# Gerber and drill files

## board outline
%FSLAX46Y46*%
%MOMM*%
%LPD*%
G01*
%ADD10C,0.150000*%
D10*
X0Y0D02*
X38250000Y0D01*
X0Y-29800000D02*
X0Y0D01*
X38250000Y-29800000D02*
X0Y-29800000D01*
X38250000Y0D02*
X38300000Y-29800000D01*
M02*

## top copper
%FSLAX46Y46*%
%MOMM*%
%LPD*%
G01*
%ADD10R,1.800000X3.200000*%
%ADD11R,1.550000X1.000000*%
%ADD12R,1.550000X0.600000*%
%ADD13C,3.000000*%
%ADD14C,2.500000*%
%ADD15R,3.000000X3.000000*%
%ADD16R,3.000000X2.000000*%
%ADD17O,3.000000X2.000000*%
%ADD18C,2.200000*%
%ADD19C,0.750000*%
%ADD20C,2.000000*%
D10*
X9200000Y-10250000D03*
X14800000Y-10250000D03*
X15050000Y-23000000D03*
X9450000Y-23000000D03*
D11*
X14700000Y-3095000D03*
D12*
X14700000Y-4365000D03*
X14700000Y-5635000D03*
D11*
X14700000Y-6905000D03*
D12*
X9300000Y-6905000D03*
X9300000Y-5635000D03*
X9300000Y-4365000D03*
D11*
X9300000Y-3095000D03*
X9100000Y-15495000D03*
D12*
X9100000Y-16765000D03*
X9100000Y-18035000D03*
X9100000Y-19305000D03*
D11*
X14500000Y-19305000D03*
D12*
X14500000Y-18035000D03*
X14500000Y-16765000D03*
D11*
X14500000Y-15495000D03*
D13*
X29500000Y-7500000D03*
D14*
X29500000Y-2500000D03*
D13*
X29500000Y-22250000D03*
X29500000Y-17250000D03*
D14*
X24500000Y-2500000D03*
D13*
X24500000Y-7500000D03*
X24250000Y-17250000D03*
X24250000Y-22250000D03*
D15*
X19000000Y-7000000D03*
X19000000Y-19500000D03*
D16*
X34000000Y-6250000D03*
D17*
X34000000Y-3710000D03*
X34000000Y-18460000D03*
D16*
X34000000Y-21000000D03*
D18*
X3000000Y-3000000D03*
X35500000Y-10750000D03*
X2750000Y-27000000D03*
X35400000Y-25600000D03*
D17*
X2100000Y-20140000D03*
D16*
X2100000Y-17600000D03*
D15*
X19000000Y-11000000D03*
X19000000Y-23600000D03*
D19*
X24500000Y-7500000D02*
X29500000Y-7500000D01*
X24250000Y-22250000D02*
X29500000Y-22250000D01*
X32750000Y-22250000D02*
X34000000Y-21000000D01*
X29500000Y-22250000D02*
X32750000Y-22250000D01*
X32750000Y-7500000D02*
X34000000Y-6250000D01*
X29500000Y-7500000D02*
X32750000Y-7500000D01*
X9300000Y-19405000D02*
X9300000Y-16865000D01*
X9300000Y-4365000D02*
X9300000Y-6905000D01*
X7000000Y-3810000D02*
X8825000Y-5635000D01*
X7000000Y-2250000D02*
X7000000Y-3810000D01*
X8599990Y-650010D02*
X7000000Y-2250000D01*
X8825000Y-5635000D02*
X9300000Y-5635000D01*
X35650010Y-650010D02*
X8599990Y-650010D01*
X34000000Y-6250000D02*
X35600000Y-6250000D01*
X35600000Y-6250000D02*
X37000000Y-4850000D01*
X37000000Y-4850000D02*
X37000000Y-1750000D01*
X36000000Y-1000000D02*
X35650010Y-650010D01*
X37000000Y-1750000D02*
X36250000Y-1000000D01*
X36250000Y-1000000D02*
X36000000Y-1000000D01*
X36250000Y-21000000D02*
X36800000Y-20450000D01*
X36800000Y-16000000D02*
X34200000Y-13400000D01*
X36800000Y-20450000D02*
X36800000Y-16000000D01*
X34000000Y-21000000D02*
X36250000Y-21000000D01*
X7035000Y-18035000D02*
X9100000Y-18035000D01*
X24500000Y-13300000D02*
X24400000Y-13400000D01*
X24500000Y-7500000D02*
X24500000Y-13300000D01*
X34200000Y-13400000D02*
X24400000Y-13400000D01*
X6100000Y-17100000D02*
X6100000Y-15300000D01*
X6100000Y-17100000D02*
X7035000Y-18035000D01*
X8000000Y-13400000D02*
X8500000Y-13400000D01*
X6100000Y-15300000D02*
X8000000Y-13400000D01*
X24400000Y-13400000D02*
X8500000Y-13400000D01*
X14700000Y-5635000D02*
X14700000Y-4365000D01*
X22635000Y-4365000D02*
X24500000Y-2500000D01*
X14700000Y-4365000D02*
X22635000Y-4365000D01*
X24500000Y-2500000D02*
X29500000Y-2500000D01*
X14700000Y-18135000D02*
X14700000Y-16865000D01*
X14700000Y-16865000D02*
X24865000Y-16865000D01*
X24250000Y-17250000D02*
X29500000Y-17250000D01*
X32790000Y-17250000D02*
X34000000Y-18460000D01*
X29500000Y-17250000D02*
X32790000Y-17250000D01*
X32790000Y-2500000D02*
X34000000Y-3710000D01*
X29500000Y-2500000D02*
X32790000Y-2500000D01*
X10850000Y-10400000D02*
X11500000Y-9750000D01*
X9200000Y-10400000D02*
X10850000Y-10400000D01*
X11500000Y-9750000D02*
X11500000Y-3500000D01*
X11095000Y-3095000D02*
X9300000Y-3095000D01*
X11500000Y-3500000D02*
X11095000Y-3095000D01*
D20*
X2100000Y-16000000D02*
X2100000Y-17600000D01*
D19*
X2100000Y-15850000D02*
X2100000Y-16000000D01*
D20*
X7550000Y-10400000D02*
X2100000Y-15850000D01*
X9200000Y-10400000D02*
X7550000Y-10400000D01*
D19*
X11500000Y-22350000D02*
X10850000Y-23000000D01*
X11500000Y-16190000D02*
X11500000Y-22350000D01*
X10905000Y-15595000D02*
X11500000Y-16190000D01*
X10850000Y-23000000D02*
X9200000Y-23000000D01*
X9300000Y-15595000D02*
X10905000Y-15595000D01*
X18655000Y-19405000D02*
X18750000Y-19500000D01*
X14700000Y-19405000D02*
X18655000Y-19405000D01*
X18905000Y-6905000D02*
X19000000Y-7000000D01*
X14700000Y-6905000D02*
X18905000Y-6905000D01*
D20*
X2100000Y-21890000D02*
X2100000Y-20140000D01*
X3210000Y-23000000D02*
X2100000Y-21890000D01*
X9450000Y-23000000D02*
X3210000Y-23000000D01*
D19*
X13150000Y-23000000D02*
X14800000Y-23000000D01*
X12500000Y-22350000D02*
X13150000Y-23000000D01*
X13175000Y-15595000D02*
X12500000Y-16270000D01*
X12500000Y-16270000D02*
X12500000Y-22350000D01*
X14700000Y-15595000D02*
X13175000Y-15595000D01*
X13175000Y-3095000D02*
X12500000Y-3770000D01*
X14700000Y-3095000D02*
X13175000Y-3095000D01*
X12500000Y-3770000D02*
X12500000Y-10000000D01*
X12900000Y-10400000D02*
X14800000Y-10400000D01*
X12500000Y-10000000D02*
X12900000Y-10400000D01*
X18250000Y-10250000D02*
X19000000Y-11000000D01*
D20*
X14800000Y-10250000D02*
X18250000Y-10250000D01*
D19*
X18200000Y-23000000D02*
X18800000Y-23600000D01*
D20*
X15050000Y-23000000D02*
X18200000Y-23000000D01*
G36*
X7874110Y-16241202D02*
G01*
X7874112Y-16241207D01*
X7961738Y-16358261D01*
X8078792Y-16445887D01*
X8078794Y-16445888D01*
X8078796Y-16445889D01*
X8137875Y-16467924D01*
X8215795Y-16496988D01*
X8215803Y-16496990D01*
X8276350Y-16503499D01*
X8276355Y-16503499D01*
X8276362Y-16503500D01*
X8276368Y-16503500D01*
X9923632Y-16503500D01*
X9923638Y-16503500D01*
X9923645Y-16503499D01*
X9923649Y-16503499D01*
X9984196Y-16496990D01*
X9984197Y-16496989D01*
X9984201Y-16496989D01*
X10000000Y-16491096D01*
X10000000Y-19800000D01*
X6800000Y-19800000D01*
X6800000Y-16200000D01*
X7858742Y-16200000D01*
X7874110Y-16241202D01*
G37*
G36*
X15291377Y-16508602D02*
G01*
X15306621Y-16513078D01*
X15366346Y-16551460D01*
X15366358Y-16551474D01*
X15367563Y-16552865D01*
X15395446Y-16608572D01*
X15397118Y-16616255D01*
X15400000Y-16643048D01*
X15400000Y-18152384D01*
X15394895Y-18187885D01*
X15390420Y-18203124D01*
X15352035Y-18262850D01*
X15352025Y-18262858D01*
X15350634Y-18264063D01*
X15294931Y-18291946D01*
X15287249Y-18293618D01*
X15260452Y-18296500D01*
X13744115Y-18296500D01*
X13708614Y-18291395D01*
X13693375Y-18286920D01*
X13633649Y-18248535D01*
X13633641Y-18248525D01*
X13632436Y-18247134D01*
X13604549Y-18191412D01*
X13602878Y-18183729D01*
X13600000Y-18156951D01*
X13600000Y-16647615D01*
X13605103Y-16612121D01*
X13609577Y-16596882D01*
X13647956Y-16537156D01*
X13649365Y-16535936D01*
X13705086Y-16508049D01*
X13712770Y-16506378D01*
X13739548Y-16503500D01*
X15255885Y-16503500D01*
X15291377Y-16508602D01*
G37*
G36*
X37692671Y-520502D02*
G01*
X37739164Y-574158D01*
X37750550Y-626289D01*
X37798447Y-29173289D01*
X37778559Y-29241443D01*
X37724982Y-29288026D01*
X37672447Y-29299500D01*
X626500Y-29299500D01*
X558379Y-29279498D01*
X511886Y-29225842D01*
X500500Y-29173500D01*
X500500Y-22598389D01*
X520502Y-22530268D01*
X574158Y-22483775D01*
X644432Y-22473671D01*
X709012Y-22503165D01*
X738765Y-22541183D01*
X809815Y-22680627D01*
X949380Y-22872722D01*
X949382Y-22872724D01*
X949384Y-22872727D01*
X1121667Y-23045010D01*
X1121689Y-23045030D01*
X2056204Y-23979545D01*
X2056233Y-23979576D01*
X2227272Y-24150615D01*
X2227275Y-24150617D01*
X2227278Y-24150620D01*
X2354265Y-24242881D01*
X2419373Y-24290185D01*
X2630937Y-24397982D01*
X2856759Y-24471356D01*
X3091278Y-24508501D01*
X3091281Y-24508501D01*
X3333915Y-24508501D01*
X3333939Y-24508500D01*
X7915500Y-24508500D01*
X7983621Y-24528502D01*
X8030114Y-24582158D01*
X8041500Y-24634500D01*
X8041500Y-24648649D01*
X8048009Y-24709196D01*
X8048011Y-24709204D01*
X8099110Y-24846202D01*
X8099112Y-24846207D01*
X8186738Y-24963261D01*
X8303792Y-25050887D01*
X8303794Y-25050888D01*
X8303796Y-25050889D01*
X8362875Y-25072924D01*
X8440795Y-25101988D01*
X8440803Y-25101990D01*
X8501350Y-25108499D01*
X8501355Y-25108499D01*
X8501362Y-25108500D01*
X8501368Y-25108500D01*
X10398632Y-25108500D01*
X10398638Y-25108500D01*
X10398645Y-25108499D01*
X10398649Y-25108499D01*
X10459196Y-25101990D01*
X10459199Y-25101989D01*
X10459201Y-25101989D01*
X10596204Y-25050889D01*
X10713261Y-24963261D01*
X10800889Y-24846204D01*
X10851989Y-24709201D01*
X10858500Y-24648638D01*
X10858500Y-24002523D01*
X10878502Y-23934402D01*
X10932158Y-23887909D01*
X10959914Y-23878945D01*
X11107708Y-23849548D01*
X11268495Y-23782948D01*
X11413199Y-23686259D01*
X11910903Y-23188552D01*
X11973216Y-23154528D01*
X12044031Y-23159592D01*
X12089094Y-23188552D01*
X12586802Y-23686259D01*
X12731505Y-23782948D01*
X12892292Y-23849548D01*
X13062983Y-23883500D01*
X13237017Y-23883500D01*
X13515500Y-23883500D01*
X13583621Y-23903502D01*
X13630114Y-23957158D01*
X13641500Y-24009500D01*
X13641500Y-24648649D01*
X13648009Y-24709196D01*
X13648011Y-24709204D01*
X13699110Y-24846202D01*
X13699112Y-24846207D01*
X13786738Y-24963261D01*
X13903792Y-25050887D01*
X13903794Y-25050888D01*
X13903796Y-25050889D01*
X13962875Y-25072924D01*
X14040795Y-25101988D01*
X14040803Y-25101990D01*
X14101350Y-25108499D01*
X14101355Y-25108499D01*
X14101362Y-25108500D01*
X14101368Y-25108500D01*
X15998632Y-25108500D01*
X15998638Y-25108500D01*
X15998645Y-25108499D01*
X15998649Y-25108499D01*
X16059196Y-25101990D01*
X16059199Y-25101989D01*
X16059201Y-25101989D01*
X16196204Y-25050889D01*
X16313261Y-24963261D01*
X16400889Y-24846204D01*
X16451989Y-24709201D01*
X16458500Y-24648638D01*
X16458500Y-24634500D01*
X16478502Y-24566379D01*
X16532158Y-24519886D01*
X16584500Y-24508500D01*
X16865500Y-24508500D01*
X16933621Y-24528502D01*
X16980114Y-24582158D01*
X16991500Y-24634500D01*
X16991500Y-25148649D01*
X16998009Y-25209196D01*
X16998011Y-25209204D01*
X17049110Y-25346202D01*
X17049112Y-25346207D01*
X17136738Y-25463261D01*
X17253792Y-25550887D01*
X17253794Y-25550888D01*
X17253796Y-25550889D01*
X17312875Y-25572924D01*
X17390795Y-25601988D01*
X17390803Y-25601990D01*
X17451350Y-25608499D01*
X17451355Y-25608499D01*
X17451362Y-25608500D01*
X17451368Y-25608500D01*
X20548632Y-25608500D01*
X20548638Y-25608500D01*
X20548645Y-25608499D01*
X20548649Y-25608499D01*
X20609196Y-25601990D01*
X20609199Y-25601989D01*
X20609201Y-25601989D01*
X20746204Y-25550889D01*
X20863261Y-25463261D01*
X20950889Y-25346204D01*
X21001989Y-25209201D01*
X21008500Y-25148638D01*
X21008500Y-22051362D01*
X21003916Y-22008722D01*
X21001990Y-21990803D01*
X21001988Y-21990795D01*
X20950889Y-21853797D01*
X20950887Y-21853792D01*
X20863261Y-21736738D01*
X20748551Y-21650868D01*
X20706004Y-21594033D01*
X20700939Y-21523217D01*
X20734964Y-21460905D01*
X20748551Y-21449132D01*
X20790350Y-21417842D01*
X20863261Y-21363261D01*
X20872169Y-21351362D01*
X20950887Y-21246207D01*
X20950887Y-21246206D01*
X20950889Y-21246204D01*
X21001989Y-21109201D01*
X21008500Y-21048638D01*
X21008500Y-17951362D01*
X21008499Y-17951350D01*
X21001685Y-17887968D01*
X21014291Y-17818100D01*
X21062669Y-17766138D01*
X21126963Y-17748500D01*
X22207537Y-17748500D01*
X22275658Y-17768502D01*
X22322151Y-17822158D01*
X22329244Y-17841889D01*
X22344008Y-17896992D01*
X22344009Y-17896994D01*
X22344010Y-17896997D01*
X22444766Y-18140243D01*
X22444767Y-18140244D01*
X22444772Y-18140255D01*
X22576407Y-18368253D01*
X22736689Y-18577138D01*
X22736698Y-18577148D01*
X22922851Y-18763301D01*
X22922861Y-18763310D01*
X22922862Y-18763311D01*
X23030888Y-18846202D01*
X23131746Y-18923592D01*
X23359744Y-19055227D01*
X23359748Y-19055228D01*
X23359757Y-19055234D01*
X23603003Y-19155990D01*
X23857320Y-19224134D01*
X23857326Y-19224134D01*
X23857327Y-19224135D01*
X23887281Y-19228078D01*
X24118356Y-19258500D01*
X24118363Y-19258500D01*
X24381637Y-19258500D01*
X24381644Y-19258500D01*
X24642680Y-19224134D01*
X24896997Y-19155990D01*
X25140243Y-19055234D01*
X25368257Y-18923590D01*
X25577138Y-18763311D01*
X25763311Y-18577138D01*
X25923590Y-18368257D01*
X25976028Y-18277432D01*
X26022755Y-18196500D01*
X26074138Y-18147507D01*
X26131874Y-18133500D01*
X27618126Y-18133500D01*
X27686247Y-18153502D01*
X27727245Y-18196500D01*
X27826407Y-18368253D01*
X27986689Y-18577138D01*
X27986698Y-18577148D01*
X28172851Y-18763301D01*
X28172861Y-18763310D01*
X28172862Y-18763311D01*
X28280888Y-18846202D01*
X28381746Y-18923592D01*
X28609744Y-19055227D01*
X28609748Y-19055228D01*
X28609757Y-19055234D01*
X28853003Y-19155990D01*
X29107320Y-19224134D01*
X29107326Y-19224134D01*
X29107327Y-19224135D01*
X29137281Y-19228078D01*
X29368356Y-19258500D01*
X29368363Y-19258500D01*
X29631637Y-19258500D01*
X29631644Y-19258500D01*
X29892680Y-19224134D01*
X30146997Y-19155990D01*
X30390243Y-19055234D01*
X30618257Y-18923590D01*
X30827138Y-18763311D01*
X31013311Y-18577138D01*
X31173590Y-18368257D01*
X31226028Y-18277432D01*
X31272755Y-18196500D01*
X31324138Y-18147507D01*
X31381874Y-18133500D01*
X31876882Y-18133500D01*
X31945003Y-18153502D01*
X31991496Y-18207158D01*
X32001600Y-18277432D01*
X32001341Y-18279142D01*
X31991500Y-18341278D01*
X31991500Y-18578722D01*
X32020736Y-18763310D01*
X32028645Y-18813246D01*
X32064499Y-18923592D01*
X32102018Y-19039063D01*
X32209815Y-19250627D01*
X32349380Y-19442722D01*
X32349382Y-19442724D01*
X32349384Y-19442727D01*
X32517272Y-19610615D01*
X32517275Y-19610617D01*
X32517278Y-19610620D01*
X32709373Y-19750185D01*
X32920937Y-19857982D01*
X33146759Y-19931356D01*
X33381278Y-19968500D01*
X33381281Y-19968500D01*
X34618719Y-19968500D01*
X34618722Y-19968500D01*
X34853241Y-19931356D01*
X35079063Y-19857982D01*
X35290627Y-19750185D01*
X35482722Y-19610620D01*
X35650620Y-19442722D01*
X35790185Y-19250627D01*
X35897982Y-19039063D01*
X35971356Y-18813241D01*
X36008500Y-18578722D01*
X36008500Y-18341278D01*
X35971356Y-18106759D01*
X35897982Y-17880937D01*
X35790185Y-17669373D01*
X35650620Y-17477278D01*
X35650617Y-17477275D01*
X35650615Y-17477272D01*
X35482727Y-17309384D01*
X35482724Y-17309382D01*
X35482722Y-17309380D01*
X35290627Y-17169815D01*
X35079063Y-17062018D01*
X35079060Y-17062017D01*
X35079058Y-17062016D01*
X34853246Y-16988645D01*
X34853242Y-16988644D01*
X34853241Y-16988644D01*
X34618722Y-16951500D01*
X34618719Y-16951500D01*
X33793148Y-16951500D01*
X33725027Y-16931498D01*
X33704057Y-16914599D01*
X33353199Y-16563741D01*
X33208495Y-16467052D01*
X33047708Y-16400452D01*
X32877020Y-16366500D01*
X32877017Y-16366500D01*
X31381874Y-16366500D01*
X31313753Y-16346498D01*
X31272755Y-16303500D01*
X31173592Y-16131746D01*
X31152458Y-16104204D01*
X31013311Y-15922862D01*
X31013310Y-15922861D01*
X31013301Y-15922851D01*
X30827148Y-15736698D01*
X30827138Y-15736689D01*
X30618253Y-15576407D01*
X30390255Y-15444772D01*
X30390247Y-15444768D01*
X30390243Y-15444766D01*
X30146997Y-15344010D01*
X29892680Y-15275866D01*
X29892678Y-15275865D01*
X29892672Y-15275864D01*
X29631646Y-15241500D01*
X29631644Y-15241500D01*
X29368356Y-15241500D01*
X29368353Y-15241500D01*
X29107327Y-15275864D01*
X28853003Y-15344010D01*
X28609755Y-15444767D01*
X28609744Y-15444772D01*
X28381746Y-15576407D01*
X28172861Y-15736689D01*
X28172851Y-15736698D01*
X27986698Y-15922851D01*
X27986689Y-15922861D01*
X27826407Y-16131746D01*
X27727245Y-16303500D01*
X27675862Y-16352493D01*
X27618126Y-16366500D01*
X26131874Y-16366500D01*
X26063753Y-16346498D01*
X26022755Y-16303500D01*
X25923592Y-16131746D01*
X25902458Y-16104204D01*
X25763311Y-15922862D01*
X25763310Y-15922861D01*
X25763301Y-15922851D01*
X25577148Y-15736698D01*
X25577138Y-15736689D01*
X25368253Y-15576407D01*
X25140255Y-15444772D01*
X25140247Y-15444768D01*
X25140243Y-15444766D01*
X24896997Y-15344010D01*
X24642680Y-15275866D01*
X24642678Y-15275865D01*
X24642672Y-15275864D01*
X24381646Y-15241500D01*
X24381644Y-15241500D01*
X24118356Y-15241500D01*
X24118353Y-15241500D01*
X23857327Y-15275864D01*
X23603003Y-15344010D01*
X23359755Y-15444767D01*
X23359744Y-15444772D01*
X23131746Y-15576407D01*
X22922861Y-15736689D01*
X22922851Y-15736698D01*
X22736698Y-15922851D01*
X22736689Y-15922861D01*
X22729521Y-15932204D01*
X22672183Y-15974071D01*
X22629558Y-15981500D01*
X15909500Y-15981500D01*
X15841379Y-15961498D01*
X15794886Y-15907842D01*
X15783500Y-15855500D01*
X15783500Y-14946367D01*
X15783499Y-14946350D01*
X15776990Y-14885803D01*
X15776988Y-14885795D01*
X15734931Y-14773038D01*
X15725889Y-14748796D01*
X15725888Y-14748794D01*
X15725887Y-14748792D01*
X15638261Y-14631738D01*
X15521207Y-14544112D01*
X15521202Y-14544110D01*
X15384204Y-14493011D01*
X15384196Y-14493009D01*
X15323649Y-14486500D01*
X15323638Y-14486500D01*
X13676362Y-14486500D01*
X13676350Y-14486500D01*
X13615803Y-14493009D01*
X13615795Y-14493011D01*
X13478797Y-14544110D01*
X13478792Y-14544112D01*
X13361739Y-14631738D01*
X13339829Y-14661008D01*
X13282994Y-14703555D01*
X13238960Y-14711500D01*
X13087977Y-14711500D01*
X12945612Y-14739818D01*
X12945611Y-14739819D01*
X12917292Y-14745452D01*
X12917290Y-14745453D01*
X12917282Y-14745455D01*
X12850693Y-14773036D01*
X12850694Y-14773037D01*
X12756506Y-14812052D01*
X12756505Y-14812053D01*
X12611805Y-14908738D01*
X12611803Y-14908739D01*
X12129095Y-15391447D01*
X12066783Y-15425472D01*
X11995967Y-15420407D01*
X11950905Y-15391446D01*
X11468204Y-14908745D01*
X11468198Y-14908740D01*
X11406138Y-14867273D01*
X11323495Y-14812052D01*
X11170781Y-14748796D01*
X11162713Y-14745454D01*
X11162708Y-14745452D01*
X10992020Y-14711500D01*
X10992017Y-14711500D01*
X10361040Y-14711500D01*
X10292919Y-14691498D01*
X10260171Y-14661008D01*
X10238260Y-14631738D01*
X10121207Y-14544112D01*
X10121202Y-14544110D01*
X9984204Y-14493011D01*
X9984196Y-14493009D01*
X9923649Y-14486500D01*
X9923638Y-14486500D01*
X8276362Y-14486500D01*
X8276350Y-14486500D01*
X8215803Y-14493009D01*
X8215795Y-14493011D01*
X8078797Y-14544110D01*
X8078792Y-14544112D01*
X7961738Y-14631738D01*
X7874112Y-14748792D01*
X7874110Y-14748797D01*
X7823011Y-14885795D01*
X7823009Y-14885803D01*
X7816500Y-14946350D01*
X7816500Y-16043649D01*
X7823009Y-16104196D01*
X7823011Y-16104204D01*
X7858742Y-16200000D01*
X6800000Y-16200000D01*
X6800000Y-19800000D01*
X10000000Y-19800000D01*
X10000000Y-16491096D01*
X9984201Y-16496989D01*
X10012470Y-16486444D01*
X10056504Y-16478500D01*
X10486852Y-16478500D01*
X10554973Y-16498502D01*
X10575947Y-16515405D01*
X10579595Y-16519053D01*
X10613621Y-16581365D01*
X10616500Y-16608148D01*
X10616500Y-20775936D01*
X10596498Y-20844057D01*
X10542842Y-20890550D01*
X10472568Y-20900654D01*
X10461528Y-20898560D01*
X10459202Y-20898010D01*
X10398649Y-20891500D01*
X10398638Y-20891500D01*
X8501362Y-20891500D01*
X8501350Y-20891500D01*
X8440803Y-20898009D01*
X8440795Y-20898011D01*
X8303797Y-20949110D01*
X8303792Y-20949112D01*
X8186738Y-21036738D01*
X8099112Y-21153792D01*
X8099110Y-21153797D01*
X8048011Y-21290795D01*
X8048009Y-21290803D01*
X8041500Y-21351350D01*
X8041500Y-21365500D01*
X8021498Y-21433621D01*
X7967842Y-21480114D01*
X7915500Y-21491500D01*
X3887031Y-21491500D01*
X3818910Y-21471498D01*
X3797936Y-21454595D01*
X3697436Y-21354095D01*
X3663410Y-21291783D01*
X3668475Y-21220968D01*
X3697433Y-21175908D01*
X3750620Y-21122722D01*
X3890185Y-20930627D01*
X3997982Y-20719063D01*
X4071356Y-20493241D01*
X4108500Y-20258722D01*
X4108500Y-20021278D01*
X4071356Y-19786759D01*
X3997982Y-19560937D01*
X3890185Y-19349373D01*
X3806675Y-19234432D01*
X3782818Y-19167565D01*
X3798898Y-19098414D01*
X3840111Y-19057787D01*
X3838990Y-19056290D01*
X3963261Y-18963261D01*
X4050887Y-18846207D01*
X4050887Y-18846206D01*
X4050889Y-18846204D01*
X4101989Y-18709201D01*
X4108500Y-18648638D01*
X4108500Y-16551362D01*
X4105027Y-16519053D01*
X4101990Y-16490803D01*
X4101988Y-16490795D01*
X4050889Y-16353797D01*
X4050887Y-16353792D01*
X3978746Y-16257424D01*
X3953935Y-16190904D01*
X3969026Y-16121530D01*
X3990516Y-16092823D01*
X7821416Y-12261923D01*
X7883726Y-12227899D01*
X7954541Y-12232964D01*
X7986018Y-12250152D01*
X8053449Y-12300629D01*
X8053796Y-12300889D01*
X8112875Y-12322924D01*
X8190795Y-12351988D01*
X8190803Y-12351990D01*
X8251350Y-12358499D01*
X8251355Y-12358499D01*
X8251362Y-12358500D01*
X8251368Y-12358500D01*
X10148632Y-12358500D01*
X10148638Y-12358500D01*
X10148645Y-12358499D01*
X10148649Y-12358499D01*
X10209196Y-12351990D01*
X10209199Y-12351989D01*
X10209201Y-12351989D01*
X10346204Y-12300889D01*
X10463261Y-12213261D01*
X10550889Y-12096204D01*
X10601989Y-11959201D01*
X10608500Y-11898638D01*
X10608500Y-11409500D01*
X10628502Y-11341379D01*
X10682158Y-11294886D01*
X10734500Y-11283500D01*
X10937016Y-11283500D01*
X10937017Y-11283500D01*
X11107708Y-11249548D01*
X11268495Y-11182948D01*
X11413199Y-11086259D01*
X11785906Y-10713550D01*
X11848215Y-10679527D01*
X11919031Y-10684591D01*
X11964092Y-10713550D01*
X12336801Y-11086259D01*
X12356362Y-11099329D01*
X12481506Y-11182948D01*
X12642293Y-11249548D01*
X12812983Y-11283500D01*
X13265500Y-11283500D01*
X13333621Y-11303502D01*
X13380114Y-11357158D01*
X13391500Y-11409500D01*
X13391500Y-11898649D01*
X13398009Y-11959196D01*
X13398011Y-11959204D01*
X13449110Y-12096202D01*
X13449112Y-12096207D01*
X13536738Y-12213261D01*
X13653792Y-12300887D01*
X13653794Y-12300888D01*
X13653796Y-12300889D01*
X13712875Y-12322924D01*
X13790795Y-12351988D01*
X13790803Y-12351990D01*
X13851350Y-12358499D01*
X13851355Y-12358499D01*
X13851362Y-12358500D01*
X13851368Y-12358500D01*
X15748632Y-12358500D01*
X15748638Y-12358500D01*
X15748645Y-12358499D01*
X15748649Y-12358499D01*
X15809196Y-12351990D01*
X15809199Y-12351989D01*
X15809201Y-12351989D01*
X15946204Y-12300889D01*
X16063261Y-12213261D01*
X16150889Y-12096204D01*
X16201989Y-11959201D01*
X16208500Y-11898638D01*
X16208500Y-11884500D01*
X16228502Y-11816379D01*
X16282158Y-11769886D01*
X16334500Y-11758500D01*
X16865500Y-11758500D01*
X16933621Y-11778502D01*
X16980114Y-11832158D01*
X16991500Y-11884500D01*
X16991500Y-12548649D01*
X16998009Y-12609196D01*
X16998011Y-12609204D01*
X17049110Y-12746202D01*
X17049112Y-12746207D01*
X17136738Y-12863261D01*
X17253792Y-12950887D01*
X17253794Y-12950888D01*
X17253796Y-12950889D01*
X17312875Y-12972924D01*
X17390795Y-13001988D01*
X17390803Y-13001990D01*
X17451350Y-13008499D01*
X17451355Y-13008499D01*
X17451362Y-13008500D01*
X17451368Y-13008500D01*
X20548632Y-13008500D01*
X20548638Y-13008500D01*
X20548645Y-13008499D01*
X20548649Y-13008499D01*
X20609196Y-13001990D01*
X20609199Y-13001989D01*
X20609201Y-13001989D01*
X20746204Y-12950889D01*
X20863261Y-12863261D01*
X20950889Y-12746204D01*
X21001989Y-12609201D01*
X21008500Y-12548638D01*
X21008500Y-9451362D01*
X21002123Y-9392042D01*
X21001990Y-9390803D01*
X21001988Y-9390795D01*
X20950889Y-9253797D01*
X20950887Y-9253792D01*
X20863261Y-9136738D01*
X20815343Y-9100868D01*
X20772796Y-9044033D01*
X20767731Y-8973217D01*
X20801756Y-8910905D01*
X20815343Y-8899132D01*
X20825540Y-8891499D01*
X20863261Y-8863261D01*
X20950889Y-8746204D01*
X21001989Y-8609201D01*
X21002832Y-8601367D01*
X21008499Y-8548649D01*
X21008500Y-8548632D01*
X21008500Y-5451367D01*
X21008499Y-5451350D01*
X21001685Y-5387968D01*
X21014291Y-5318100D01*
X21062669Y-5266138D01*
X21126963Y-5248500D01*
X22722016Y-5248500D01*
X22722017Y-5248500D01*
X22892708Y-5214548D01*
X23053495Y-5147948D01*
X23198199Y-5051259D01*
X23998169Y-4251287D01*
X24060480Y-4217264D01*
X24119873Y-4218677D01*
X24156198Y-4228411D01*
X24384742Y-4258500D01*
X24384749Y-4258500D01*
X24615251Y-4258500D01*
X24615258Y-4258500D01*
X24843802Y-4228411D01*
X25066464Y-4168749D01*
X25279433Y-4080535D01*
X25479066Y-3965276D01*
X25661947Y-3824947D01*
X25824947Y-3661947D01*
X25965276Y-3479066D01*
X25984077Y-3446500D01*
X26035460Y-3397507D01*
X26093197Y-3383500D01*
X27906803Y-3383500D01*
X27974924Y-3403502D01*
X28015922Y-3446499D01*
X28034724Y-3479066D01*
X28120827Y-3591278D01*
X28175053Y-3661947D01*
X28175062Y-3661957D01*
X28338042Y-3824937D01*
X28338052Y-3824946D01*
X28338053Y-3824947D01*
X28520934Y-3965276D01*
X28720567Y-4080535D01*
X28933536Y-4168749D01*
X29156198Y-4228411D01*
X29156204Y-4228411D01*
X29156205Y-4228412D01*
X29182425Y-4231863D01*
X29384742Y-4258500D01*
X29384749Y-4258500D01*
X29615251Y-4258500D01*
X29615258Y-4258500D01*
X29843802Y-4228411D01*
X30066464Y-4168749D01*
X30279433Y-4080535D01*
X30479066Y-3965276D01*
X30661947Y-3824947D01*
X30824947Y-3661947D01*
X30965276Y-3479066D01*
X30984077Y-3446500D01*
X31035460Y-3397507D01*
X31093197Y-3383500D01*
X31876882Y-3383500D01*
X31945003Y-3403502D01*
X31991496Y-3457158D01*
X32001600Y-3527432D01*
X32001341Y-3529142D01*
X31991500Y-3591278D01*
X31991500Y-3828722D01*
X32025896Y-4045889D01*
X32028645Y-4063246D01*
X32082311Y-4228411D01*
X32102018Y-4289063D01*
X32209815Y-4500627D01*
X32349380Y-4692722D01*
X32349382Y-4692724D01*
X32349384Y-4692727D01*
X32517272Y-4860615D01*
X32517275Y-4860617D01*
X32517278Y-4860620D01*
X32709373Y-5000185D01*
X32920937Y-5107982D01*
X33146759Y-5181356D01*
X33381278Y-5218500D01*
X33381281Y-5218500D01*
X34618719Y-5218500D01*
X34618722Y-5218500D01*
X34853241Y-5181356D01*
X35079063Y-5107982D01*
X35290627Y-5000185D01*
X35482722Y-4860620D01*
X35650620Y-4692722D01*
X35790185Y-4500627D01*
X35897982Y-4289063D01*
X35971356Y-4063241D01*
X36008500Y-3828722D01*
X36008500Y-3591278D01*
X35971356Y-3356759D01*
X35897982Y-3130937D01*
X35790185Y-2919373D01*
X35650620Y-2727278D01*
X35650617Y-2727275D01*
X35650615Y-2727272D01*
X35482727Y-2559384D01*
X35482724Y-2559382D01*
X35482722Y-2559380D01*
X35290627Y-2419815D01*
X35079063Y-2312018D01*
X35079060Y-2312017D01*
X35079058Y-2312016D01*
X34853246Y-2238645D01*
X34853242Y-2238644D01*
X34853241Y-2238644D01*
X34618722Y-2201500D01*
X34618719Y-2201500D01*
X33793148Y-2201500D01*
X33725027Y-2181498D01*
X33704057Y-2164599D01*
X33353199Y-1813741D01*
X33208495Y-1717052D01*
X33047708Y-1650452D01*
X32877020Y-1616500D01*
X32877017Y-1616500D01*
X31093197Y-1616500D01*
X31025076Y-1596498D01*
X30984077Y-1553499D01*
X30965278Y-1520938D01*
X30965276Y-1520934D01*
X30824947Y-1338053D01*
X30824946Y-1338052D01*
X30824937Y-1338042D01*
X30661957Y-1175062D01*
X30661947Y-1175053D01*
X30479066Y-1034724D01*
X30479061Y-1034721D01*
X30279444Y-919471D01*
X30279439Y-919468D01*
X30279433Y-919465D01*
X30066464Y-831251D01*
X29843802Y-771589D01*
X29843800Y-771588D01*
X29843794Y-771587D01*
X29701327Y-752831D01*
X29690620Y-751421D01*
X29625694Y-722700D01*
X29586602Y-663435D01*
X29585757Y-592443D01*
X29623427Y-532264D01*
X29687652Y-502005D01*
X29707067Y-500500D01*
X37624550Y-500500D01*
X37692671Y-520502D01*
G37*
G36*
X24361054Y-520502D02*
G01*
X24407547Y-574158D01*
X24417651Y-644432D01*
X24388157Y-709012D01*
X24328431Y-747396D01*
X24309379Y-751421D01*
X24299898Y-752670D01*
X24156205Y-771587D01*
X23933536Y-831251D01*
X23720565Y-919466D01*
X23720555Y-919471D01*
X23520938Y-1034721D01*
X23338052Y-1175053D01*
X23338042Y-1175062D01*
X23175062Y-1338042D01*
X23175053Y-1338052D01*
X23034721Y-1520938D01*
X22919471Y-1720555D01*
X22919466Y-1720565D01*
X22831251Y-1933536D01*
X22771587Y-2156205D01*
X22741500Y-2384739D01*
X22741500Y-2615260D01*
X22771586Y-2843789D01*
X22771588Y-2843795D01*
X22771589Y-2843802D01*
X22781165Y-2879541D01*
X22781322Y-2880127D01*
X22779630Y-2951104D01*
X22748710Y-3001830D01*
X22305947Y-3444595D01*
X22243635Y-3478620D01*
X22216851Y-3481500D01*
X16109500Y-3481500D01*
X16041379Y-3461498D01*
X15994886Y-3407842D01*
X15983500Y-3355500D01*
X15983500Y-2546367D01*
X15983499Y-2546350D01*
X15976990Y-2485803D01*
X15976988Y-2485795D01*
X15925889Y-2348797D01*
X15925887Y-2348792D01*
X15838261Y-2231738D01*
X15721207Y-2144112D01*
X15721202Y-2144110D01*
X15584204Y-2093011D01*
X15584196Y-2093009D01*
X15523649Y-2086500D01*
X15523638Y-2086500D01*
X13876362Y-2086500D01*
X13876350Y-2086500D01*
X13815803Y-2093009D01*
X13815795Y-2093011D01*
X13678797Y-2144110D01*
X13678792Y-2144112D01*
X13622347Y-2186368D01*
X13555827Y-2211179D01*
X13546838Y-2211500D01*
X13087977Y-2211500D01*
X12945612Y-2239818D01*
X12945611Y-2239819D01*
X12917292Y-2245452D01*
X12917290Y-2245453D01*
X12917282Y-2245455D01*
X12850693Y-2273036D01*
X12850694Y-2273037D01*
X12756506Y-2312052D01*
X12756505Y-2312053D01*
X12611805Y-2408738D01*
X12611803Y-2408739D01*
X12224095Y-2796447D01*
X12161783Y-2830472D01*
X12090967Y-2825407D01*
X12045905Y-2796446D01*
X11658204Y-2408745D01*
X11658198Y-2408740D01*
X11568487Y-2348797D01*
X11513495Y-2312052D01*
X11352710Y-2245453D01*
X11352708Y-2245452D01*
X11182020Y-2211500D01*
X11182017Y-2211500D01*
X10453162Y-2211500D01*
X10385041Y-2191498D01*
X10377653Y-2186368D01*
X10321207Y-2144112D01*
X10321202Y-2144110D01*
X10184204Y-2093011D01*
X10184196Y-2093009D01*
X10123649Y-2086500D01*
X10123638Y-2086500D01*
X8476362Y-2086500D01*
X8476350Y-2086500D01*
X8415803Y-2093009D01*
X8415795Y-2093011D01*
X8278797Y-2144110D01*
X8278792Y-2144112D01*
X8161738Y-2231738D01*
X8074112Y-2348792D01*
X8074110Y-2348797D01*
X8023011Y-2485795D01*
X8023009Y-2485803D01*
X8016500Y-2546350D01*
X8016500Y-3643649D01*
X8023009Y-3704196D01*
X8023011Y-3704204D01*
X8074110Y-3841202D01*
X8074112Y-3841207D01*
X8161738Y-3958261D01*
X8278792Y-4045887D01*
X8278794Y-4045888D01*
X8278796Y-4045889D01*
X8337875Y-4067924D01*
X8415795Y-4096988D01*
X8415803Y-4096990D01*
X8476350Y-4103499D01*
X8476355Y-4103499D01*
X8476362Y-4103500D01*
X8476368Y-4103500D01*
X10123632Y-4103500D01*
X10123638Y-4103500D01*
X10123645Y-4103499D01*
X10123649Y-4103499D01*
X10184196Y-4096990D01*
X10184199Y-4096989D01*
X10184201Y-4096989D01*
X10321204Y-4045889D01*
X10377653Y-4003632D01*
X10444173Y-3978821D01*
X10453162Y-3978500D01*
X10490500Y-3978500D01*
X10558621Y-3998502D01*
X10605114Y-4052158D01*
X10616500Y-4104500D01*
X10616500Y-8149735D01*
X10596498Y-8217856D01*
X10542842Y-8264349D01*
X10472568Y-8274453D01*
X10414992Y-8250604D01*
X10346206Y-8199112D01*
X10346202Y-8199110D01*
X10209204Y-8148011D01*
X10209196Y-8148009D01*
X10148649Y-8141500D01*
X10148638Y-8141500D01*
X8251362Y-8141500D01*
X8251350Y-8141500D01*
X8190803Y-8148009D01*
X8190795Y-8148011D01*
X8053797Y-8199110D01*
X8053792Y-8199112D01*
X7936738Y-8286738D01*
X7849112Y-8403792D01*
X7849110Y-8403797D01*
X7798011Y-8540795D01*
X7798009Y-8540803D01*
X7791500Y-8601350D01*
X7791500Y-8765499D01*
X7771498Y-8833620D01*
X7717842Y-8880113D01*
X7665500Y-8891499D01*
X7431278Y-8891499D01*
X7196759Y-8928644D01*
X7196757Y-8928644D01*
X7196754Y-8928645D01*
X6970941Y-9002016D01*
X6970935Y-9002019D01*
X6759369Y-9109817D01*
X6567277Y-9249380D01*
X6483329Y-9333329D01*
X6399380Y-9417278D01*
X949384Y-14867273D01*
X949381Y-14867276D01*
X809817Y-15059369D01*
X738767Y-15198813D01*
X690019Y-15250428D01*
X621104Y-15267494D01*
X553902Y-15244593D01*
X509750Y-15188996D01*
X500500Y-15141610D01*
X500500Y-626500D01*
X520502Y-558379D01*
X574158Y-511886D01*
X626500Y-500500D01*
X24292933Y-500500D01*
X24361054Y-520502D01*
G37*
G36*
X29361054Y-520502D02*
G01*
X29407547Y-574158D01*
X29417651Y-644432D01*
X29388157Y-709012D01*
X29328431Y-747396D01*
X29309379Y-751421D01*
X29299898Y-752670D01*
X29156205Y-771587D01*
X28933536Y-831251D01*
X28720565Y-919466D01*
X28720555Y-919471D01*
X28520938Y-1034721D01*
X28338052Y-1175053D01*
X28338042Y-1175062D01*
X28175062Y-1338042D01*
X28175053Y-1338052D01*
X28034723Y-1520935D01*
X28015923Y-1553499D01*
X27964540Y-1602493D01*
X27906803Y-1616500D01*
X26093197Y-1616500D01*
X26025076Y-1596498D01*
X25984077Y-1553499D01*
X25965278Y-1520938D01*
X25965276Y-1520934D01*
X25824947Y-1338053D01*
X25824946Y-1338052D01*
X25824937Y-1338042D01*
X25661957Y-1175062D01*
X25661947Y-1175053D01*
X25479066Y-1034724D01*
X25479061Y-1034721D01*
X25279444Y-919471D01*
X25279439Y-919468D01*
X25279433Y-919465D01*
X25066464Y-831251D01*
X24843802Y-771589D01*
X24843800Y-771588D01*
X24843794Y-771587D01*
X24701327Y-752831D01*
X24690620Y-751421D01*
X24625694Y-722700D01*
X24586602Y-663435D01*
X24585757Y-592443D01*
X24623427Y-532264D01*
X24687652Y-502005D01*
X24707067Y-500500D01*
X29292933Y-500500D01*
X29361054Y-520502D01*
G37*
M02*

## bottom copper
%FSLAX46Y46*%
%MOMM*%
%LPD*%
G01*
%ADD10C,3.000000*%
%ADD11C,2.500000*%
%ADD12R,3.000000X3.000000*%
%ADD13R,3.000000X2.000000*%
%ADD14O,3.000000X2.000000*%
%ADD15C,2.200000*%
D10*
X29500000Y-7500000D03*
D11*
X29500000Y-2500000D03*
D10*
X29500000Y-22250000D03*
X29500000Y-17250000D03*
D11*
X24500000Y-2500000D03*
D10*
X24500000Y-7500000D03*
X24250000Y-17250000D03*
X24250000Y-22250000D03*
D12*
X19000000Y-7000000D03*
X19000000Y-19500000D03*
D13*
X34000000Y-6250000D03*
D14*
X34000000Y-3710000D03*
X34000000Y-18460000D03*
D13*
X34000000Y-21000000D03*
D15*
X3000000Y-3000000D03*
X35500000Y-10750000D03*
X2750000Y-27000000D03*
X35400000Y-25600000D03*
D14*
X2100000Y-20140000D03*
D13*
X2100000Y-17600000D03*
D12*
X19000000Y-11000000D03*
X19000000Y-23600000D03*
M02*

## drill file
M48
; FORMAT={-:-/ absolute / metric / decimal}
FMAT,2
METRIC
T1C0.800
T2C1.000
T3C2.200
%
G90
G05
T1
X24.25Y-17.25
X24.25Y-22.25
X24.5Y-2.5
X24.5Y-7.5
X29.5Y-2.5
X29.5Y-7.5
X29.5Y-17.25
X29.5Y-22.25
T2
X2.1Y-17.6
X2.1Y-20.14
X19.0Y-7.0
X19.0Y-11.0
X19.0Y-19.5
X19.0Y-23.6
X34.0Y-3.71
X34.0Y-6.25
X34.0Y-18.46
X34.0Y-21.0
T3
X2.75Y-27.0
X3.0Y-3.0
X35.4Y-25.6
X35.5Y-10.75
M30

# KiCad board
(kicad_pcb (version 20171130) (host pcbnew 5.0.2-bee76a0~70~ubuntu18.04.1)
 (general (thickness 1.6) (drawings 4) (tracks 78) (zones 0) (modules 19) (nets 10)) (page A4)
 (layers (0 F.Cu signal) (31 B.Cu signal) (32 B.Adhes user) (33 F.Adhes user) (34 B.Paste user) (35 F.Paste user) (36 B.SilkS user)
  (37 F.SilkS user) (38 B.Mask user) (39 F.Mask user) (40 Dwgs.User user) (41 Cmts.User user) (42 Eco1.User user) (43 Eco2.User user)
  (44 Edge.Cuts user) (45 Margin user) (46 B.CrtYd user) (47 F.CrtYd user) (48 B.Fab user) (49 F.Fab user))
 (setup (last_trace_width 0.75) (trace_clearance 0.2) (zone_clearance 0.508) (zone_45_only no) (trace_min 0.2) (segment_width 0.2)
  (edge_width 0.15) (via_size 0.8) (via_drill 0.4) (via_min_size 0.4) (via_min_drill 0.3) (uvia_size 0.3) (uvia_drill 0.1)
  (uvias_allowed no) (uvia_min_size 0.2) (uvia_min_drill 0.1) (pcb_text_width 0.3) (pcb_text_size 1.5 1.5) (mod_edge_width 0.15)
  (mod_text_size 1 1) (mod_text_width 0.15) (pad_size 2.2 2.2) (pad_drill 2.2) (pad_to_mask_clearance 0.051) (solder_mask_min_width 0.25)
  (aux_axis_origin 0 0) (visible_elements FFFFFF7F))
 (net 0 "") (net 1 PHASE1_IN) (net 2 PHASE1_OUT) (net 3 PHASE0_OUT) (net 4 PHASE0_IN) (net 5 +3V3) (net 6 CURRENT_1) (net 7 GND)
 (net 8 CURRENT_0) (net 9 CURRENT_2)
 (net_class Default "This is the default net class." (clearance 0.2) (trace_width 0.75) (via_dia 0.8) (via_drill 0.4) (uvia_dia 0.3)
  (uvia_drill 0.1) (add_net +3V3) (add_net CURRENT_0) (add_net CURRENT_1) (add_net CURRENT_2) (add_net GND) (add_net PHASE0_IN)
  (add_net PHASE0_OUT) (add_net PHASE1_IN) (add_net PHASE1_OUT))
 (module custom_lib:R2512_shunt (layer F.Cu) (at 12 10.25 180)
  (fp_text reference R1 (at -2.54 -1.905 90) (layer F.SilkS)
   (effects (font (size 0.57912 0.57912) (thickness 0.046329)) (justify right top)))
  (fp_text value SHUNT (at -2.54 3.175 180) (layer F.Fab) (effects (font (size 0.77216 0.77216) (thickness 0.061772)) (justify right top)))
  (pad 2 smd rect (at 2.8 0 180) (size 1.8 3.2) (layers F.Cu F.Paste F.Mask) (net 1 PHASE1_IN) (solder_mask_margin 0.075))
  (pad 1 smd rect (at -2.8 0 180) (size 1.8 3.2) (layers F.Cu F.Paste F.Mask) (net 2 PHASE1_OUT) (solder_mask_margin 0.075)))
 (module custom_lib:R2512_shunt (layer F.Cu) (at 12.25 23 180)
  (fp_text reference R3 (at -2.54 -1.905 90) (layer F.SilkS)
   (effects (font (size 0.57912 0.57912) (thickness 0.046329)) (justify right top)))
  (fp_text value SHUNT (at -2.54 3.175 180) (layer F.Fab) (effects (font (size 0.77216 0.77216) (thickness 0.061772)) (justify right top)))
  (pad 1 smd rect (at -2.8 0 180) (size 1.8 3.2) (layers F.Cu F.Paste F.Mask) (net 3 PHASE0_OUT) (solder_mask_margin 0.075))
  (pad 2 smd rect (at 2.8 0 180) (size 1.8 3.2) (layers F.Cu F.Paste F.Mask) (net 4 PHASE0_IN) (solder_mask_margin 0.075)))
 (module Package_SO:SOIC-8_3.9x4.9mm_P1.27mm (layer F.Cu) (at 12 5)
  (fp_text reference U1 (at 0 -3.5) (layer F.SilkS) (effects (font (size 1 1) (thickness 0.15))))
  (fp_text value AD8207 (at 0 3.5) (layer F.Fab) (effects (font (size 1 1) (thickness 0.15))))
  (pad 8 smd rect (at 2.7 -1.905) (size 1.55 1) (layers F.Cu F.Paste F.Mask) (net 2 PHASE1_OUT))
  (pad 7 smd rect (at 2.7 -0.635) (size 1.55 0.6) (layers F.Cu F.Paste F.Mask) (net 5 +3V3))
  (pad 6 smd rect (at 2.7 0.635) (size 1.55 0.6) (layers F.Cu F.Paste F.Mask) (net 5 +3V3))
  (pad 5 smd rect (at 2.7 1.905) (size 1.55 1) (layers F.Cu F.Paste F.Mask) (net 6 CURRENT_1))
  (pad 4 smd rect (at -2.7 1.905) (size 1.55 0.6) (layers F.Cu F.Paste F.Mask) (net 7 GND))
  (pad 3 smd rect (at -2.7 0.635) (size 1.55 0.6) (layers F.Cu F.Paste F.Mask) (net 7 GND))
  (pad 2 smd rect (at -2.7 -0.635) (size 1.55 0.6) (layers F.Cu F.Paste F.Mask) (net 7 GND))
  (pad 1 smd rect (at -2.7 -1.905) (size 1.55 1) (layers F.Cu F.Paste F.Mask) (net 1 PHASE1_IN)))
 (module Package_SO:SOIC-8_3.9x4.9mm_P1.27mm (layer F.Cu) (at 11.8 17.4)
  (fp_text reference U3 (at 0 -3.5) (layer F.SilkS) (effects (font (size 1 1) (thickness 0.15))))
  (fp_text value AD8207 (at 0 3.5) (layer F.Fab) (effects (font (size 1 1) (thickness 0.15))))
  (pad 1 smd rect (at -2.7 -1.905) (size 1.55 1) (layers F.Cu F.Paste F.Mask) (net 4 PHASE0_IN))
  (pad 2 smd rect (at -2.7 -0.635) (size 1.55 0.6) (layers F.Cu F.Paste F.Mask) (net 7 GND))
  (pad 3 smd rect (at -2.7 0.635) (size 1.55 0.6) (layers F.Cu F.Paste F.Mask) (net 7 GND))
  (pad 4 smd rect (at -2.7 1.905) (size 1.55 0.6) (layers F.Cu F.Paste F.Mask) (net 7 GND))
  (pad 5 smd rect (at 2.7 1.905) (size 1.55 1) (layers F.Cu F.Paste F.Mask) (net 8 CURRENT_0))
  (pad 6 smd rect (at 2.7 0.635) (size 1.55 0.6) (layers F.Cu F.Paste F.Mask) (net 5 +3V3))
  (pad 7 smd rect (at 2.7 -0.635) (size 1.55 0.6) (layers F.Cu F.Paste F.Mask) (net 5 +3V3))
  (pad 8 smd rect (at 2.7 -1.905) (size 1.55 1) (layers F.Cu F.Paste F.Mask) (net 3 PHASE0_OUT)))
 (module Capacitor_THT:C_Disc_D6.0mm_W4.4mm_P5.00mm (layer F.Cu) (at 29.5 7.5 90)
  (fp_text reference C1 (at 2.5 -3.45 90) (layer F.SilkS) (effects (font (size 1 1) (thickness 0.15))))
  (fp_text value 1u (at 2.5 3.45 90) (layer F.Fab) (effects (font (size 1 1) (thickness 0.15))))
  (pad 1 thru_hole circle (at 0 0 90) (size 3 3) (drill 0.8) (layers *.Cu *.Mask) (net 7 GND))
  (pad 2 thru_hole circle (at 5 0 90) (size 2.5 2.5) (drill 0.8) (layers *.Cu *.Mask) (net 5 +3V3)))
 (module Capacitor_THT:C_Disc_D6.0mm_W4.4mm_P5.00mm (layer F.Cu) (at 29.5 22.25 90)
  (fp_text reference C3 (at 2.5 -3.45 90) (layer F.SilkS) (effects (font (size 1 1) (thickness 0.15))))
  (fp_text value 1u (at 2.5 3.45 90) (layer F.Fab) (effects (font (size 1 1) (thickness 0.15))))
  (pad 1 thru_hole circle (at 0 0 90) (size 3 3) (drill 0.8) (layers *.Cu *.Mask) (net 7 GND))
  (pad 2 thru_hole circle (at 5 0 90) (size 3 3) (drill 0.8) (layers *.Cu *.Mask) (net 5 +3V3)))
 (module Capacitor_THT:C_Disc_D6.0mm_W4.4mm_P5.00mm (layer F.Cu) (at 24.5 7.5 90)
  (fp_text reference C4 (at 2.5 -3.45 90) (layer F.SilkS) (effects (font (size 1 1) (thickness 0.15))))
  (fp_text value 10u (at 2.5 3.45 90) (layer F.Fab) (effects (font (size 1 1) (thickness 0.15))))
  (pad 2 thru_hole circle (at 5 0 90) (size 2.5 2.5) (drill 0.8) (layers *.Cu *.Mask) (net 5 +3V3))
  (pad 1 thru_hole circle (at 0 0 90) (size 3 3) (drill 0.8) (layers *.Cu *.Mask) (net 7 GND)))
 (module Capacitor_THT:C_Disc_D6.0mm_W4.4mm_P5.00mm (layer F.Cu) (at 24.25 22.25 90)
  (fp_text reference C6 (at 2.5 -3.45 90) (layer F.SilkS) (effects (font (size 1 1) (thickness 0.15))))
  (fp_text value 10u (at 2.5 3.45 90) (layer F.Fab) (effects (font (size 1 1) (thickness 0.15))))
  (pad 2 thru_hole circle (at 5 0 90) (size 3 3) (drill 0.8) (layers *.Cu *.Mask) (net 5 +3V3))
  (pad 1 thru_hole circle (at 0 0 90) (size 3 3) (drill 0.8) (layers *.Cu *.Mask) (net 7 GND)))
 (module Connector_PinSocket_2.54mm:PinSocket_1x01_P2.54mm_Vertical (layer F.Cu) (at 19 7)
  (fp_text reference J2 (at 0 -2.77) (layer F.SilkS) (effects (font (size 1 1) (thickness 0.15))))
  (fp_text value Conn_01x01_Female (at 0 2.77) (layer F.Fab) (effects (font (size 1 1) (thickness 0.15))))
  (pad 1 thru_hole rect (at 0 0) (size 3 3) (drill 1) (layers *.Cu *.Mask) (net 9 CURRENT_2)))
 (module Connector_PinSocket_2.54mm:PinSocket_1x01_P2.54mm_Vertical (layer F.Cu) (at 19 19.5)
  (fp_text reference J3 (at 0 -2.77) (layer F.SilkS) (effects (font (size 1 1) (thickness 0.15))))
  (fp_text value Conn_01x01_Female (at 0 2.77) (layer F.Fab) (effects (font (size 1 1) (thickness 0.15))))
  (pad 1 thru_hole rect (at 0 0) (size 3 3) (drill 1) (layers *.Cu *.Mask) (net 6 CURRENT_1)))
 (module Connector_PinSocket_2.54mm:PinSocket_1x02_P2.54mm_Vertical (layer F.Cu) (at 34 6.25 180)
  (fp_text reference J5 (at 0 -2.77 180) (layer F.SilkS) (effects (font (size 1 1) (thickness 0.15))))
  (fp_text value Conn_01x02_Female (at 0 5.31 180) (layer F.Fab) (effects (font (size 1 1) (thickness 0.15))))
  (pad 1 thru_hole rect (at 0 0 180) (size 3 2) (drill 1) (layers *.Cu *.Mask) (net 7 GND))
  (pad 2 thru_hole oval (at 0 2.54 180) (size 3 2) (drill 1) (layers *.Cu *.Mask) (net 5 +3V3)))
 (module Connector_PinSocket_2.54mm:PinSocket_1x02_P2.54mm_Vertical (layer F.Cu) (at 34 21 180)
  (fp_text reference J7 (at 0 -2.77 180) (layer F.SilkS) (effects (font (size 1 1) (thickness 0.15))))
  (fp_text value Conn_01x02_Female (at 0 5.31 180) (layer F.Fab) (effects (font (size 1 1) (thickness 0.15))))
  (pad 2 thru_hole oval (at 0 2.54 180) (size 3 2) (drill 1) (layers *.Cu *.Mask) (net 5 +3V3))
  (pad 1 thru_hole rect (at 0 0 180) (size 3 2) (drill 1) (layers *.Cu *.Mask) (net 7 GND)))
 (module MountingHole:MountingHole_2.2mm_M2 (layer F.Cu) (at 3 3)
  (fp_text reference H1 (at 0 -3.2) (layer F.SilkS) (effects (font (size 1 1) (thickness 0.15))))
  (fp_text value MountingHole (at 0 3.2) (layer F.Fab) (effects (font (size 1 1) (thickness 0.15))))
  (pad 1 thru_hole circle (at 0 0) (size 2.2 2.2) (drill 2.2) (layers *.Cu *.Mask) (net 7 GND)))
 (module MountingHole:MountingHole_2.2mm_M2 (layer F.Cu) (at 35.5 10.75)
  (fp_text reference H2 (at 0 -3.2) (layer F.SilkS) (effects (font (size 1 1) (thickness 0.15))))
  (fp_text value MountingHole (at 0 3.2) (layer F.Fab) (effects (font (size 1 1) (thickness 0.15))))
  (pad 1 thru_hole circle (at 0 0) (size 2.2 2.2) (drill 2.2) (layers *.Cu *.Mask) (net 7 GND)))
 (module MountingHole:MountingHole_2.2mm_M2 (layer F.Cu) (at 2.75 27)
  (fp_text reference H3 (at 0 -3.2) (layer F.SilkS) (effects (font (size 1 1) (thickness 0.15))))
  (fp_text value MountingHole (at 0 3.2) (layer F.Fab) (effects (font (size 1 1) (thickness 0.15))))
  (pad 1 thru_hole circle (at 0 0) (size 2.2 2.2) (drill 2.2) (layers *.Cu *.Mask) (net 7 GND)))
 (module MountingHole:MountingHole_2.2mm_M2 (layer F.Cu) (at 35.4 25.6)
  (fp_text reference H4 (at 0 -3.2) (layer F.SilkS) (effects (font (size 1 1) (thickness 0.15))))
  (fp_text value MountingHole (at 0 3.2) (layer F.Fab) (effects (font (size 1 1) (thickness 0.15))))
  (pad 1 thru_hole circle (at 0 0) (size 2.2 2.2) (drill 2.2) (layers *.Cu *.Mask) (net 7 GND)))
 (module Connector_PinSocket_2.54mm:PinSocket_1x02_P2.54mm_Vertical (layer F.Cu) (at 2.1 17.6)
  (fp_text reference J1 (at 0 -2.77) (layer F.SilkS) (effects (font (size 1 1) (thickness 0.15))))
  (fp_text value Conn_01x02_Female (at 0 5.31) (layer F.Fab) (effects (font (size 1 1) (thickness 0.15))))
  (pad 2 thru_hole oval (at 0 2.54) (size 3 2) (drill 1) (layers *.Cu *.Mask) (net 4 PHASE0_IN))
  (pad 1 thru_hole rect (at 0 0) (size 3 2) (drill 1) (layers *.Cu *.Mask) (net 1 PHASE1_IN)))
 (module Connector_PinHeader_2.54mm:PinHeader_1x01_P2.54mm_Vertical (layer F.Cu) (at 19 11)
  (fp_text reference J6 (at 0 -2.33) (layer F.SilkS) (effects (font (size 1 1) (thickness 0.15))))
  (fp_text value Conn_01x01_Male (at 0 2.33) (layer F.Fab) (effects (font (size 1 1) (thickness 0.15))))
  (pad 1 thru_hole rect (at 0 0) (size 3 3) (drill 1) (layers *.Cu *.Mask) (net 2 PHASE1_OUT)))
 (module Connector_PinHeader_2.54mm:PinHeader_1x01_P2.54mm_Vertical (layer F.Cu) (at 19 23.6 180)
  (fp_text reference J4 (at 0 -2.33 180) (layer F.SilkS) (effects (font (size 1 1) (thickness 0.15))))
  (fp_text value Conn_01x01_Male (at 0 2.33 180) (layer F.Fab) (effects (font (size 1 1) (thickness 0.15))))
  (pad 1 thru_hole rect (at 0 0 180) (size 3 3) (drill 1) (layers *.Cu *.Mask) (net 3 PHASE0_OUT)))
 (gr_line (start 0 0) (end 38.25 0) (layer Edge.Cuts) (width 0.15))
 (gr_line (start 0 29.8) (end 0 0) (layer Edge.Cuts) (width 0.15))
 (gr_line (start 38.25 29.8) (end 0 29.8) (layer Edge.Cuts) (width 0.15))
 (gr_line (start 38.25 0) (end 38.3 29.8) (layer Edge.Cuts) (width 0.15))
 (segment (start 24.5 7.5) (end 29.5 7.5) (width 0.75) (layer F.Cu) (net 7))
 (segment (start 24.25 22.25) (end 29.5 22.25) (width 0.75) (layer F.Cu) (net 7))
 (segment (start 32.75 22.25) (end 34 21) (width 0.75) (layer F.Cu) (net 7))
 (segment (start 29.5 22.25) (end 32.75 22.25) (width 0.75) (layer F.Cu) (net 7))
 (segment (start 32.75 7.5) (end 34 6.25) (width 0.75) (layer F.Cu) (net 7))
 (segment (start 29.5 7.5) (end 32.75 7.5) (width 0.75) (layer F.Cu) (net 7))
 (segment (start 9.3 19.405) (end 9.3 16.865) (width 0.75) (layer F.Cu) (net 7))
 (segment (start 9.3 4.365) (end 9.3 6.905) (width 0.75) (layer F.Cu) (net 7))
 (segment (start 7 3.81) (end 8.825 5.635) (width 0.75) (layer F.Cu) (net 7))
 (segment (start 7 2.25) (end 7 3.81) (width 0.75) (layer F.Cu) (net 7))
 (segment (start 8.59999 0.65001) (end 7 2.25) (width 0.75) (layer F.Cu) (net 7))
 (segment (start 8.825 5.635) (end 9.3 5.635) (width 0.75) (layer F.Cu) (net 7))
 (segment (start 35.65001 0.65001) (end 8.59999 0.65001) (width 0.75) (layer F.Cu) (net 7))
 (segment (start 34 6.25) (end 35.6 6.25) (width 0.75) (layer F.Cu) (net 7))
 (segment (start 35.6 6.25) (end 37 4.85) (width 0.75) (layer F.Cu) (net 7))
 (segment (start 37 4.85) (end 37 1.75) (width 0.75) (layer F.Cu) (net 7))
 (segment (start 36 1) (end 35.65001 0.65001) (width 0.75) (layer F.Cu) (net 7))
 (segment (start 37 1.75) (end 36.25 1) (width 0.75) (layer F.Cu) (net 7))
 (segment (start 36.25 1) (end 36 1) (width 0.75) (layer F.Cu) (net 7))
 (segment (start 36.25 21) (end 36.8 20.45) (width 0.75) (layer F.Cu) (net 7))
 (segment (start 36.8 16) (end 34.2 13.4) (width 0.75) (layer F.Cu) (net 7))
 (segment (start 36.8 20.45) (end 36.8 16) (width 0.75) (layer F.Cu) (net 7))
 (segment (start 34 21) (end 36.25 21) (width 0.75) (layer F.Cu) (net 7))
 (segment (start 7.035 18.035) (end 9.1 18.035) (width 0.75) (layer F.Cu) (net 7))
 (segment (start 24.5 13.3) (end 24.4 13.4) (width 0.75) (layer F.Cu) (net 7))
 (segment (start 24.5 7.5) (end 24.5 13.3) (width 0.75) (layer F.Cu) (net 7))
 (segment (start 34.2 13.4) (end 24.4 13.4) (width 0.75) (layer F.Cu) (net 7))
 (segment (start 6.1 17.1) (end 6.1 15.3) (width 0.75) (layer F.Cu) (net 7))
 (segment (start 6.1 17.1) (end 7.035 18.035) (width 0.75) (layer F.Cu) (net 7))
 (segment (start 8 13.4) (end 8.5 13.4) (width 0.75) (layer F.Cu) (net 7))
 (segment (start 6.1 15.3) (end 8 13.4) (width 0.75) (layer F.Cu) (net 7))
 (segment (start 24.4 13.4) (end 8.5 13.4) (width 0.75) (layer F.Cu) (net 7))
 (segment (start 14.7 5.635) (end 14.7 4.365) (width 0.75) (layer F.Cu) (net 5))
 (segment (start 22.635 4.365) (end 24.5 2.5) (width 0.75) (layer F.Cu) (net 5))
 (segment (start 14.7 4.365) (end 22.635 4.365) (width 0.75) (layer F.Cu) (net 5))
 (segment (start 24.5 2.5) (end 29.5 2.5) (width 0.75) (layer F.Cu) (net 5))
 (segment (start 14.7 18.135) (end 14.7 16.865) (width 0.75) (layer F.Cu) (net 5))
 (segment (start 14.7 16.865) (end 24.865 16.865) (width 0.75) (layer F.Cu) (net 5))
 (segment (start 24.25 17.25) (end 29.5 17.25) (width 0.75) (layer F.Cu) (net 5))
 (segment (start 32.79 17.25) (end 34 18.46) (width 0.75) (layer F.Cu) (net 5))
 (segment (start 29.5 17.25) (end 32.79 17.25) (width 0.75) (layer F.Cu) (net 5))
 (segment (start 32.79 2.5) (end 34 3.71) (width 0.75) (layer F.Cu) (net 5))
 (segment (start 29.5 2.5) (end 32.79 2.5) (width 0.75) (layer F.Cu) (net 5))
 (segment (start 10.85 10.4) (end 11.5 9.75) (width 0.75) (layer F.Cu) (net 1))
 (segment (start 9.2 10.4) (end 10.85 10.4) (width 0.75) (layer F.Cu) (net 1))
 (segment (start 11.5 9.75) (end 11.5 3.5) (width 0.75) (layer F.Cu) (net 1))
 (segment (start 11.095 3.095) (end 9.3 3.095) (width 0.75) (layer F.Cu) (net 1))
 (segment (start 11.5 3.5) (end 11.095 3.095) (width 0.75) (layer F.Cu) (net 1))
 (segment (start 2.1 16) (end 2.1 17.6) (width 2) (layer F.Cu) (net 1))
 (segment (start 2.1 15.85) (end 2.1 16) (width 0.75) (layer F.Cu) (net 1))
 (segment (start 7.55 10.4) (end 2.1 15.85) (width 2) (layer F.Cu) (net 1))
 (segment (start 9.2 10.4) (end 7.55 10.4) (width 2) (layer F.Cu) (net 1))
 (segment (start 11.5 22.35) (end 10.85 23) (width 0.75) (layer F.Cu) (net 4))
 (segment (start 11.5 16.19) (end 11.5 22.35) (width 0.75) (layer F.Cu) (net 4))
 (segment (start 10.905 15.595) (end 11.5 16.19) (width 0.75) (layer F.Cu) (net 4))
 (segment (start 10.85 23) (end 9.2 23) (width 0.75) (layer F.Cu) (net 4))
 (segment (start 9.3 15.595) (end 10.905 15.595) (width 0.75) (layer F.Cu) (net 4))
 (segment (start 18.655 19.405) (end 18.75 19.5) (width 0.75) (layer F.Cu) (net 6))
 (segment (start 14.7 19.405) (end 18.655 19.405) (width 0.75) (layer F.Cu) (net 6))
 (segment (start 18.905 6.905) (end 19 7) (width 0.75) (layer F.Cu) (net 9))
 (segment (start 14.7 6.905) (end 18.905 6.905) (width 0.75) (layer F.Cu) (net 9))
 (segment (start 2.1 21.89) (end 2.1 20.14) (width 2) (layer F.Cu) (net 4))
 (segment (start 3.21 23) (end 2.1 21.89) (width 2) (layer F.Cu) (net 4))
 (segment (start 9.45 23) (end 3.21 23) (width 2) (layer F.Cu) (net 4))
 (segment (start 13.15 23) (end 14.8 23) (width 0.75) (layer F.Cu) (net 3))
 (segment (start 12.5 22.35) (end 13.15 23) (width 0.75) (layer F.Cu) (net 3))
 (segment (start 13.175 15.595) (end 12.5 16.27) (width 0.75) (layer F.Cu) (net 3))
 (segment (start 12.5 16.27) (end 12.5 22.35) (width 0.75) (layer F.Cu) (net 3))
 (segment (start 14.7 15.595) (end 13.175 15.595) (width 0.75) (layer F.Cu) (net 3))
 (segment (start 13.175 3.095) (end 12.5 3.77) (width 0.75) (layer F.Cu) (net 2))
 (segment (start 14.7 3.095) (end 13.175 3.095) (width 0.75) (layer F.Cu) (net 2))
 (segment (start 12.5 3.77) (end 12.5 10) (width 0.75) (layer F.Cu) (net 2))
 (segment (start 12.9 10.4) (end 14.8 10.4) (width 0.75) (layer F.Cu) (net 2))
 (segment (start 12.5 10) (end 12.9 10.4) (width 0.75) (layer F.Cu) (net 2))
 (segment (start 18.25 10.25) (end 19 11) (width 0.75) (layer F.Cu) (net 2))
 (segment (start 14.8 10.25) (end 18.25 10.25) (width 2) (layer F.Cu) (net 2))
 (segment (start 18.2 23) (end 18.8 23.6) (width 0.75) (layer F.Cu) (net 3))
 (segment (start 15.05 23) (end 18.2 23) (width 2) (layer F.Cu) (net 3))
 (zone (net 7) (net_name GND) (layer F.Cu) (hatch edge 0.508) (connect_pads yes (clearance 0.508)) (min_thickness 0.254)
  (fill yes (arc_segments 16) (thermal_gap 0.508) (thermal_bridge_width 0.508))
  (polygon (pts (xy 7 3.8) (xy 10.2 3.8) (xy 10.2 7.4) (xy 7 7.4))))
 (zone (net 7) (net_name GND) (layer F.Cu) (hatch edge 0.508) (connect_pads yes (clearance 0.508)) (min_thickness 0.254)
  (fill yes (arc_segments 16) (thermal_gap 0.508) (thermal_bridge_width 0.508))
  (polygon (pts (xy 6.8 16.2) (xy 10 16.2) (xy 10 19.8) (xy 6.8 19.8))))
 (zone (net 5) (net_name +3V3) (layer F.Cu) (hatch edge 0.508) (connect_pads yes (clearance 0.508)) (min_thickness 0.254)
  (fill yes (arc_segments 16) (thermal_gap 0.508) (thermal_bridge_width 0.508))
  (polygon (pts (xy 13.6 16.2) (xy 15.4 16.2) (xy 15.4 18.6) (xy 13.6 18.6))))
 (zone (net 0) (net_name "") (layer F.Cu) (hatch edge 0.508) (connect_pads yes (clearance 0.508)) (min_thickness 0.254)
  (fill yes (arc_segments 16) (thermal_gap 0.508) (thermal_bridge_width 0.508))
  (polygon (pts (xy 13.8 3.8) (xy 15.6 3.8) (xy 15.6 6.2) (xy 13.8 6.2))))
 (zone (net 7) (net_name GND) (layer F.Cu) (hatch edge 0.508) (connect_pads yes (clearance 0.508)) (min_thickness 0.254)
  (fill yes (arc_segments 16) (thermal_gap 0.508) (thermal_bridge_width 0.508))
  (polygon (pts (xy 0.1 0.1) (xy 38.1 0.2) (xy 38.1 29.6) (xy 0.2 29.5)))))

